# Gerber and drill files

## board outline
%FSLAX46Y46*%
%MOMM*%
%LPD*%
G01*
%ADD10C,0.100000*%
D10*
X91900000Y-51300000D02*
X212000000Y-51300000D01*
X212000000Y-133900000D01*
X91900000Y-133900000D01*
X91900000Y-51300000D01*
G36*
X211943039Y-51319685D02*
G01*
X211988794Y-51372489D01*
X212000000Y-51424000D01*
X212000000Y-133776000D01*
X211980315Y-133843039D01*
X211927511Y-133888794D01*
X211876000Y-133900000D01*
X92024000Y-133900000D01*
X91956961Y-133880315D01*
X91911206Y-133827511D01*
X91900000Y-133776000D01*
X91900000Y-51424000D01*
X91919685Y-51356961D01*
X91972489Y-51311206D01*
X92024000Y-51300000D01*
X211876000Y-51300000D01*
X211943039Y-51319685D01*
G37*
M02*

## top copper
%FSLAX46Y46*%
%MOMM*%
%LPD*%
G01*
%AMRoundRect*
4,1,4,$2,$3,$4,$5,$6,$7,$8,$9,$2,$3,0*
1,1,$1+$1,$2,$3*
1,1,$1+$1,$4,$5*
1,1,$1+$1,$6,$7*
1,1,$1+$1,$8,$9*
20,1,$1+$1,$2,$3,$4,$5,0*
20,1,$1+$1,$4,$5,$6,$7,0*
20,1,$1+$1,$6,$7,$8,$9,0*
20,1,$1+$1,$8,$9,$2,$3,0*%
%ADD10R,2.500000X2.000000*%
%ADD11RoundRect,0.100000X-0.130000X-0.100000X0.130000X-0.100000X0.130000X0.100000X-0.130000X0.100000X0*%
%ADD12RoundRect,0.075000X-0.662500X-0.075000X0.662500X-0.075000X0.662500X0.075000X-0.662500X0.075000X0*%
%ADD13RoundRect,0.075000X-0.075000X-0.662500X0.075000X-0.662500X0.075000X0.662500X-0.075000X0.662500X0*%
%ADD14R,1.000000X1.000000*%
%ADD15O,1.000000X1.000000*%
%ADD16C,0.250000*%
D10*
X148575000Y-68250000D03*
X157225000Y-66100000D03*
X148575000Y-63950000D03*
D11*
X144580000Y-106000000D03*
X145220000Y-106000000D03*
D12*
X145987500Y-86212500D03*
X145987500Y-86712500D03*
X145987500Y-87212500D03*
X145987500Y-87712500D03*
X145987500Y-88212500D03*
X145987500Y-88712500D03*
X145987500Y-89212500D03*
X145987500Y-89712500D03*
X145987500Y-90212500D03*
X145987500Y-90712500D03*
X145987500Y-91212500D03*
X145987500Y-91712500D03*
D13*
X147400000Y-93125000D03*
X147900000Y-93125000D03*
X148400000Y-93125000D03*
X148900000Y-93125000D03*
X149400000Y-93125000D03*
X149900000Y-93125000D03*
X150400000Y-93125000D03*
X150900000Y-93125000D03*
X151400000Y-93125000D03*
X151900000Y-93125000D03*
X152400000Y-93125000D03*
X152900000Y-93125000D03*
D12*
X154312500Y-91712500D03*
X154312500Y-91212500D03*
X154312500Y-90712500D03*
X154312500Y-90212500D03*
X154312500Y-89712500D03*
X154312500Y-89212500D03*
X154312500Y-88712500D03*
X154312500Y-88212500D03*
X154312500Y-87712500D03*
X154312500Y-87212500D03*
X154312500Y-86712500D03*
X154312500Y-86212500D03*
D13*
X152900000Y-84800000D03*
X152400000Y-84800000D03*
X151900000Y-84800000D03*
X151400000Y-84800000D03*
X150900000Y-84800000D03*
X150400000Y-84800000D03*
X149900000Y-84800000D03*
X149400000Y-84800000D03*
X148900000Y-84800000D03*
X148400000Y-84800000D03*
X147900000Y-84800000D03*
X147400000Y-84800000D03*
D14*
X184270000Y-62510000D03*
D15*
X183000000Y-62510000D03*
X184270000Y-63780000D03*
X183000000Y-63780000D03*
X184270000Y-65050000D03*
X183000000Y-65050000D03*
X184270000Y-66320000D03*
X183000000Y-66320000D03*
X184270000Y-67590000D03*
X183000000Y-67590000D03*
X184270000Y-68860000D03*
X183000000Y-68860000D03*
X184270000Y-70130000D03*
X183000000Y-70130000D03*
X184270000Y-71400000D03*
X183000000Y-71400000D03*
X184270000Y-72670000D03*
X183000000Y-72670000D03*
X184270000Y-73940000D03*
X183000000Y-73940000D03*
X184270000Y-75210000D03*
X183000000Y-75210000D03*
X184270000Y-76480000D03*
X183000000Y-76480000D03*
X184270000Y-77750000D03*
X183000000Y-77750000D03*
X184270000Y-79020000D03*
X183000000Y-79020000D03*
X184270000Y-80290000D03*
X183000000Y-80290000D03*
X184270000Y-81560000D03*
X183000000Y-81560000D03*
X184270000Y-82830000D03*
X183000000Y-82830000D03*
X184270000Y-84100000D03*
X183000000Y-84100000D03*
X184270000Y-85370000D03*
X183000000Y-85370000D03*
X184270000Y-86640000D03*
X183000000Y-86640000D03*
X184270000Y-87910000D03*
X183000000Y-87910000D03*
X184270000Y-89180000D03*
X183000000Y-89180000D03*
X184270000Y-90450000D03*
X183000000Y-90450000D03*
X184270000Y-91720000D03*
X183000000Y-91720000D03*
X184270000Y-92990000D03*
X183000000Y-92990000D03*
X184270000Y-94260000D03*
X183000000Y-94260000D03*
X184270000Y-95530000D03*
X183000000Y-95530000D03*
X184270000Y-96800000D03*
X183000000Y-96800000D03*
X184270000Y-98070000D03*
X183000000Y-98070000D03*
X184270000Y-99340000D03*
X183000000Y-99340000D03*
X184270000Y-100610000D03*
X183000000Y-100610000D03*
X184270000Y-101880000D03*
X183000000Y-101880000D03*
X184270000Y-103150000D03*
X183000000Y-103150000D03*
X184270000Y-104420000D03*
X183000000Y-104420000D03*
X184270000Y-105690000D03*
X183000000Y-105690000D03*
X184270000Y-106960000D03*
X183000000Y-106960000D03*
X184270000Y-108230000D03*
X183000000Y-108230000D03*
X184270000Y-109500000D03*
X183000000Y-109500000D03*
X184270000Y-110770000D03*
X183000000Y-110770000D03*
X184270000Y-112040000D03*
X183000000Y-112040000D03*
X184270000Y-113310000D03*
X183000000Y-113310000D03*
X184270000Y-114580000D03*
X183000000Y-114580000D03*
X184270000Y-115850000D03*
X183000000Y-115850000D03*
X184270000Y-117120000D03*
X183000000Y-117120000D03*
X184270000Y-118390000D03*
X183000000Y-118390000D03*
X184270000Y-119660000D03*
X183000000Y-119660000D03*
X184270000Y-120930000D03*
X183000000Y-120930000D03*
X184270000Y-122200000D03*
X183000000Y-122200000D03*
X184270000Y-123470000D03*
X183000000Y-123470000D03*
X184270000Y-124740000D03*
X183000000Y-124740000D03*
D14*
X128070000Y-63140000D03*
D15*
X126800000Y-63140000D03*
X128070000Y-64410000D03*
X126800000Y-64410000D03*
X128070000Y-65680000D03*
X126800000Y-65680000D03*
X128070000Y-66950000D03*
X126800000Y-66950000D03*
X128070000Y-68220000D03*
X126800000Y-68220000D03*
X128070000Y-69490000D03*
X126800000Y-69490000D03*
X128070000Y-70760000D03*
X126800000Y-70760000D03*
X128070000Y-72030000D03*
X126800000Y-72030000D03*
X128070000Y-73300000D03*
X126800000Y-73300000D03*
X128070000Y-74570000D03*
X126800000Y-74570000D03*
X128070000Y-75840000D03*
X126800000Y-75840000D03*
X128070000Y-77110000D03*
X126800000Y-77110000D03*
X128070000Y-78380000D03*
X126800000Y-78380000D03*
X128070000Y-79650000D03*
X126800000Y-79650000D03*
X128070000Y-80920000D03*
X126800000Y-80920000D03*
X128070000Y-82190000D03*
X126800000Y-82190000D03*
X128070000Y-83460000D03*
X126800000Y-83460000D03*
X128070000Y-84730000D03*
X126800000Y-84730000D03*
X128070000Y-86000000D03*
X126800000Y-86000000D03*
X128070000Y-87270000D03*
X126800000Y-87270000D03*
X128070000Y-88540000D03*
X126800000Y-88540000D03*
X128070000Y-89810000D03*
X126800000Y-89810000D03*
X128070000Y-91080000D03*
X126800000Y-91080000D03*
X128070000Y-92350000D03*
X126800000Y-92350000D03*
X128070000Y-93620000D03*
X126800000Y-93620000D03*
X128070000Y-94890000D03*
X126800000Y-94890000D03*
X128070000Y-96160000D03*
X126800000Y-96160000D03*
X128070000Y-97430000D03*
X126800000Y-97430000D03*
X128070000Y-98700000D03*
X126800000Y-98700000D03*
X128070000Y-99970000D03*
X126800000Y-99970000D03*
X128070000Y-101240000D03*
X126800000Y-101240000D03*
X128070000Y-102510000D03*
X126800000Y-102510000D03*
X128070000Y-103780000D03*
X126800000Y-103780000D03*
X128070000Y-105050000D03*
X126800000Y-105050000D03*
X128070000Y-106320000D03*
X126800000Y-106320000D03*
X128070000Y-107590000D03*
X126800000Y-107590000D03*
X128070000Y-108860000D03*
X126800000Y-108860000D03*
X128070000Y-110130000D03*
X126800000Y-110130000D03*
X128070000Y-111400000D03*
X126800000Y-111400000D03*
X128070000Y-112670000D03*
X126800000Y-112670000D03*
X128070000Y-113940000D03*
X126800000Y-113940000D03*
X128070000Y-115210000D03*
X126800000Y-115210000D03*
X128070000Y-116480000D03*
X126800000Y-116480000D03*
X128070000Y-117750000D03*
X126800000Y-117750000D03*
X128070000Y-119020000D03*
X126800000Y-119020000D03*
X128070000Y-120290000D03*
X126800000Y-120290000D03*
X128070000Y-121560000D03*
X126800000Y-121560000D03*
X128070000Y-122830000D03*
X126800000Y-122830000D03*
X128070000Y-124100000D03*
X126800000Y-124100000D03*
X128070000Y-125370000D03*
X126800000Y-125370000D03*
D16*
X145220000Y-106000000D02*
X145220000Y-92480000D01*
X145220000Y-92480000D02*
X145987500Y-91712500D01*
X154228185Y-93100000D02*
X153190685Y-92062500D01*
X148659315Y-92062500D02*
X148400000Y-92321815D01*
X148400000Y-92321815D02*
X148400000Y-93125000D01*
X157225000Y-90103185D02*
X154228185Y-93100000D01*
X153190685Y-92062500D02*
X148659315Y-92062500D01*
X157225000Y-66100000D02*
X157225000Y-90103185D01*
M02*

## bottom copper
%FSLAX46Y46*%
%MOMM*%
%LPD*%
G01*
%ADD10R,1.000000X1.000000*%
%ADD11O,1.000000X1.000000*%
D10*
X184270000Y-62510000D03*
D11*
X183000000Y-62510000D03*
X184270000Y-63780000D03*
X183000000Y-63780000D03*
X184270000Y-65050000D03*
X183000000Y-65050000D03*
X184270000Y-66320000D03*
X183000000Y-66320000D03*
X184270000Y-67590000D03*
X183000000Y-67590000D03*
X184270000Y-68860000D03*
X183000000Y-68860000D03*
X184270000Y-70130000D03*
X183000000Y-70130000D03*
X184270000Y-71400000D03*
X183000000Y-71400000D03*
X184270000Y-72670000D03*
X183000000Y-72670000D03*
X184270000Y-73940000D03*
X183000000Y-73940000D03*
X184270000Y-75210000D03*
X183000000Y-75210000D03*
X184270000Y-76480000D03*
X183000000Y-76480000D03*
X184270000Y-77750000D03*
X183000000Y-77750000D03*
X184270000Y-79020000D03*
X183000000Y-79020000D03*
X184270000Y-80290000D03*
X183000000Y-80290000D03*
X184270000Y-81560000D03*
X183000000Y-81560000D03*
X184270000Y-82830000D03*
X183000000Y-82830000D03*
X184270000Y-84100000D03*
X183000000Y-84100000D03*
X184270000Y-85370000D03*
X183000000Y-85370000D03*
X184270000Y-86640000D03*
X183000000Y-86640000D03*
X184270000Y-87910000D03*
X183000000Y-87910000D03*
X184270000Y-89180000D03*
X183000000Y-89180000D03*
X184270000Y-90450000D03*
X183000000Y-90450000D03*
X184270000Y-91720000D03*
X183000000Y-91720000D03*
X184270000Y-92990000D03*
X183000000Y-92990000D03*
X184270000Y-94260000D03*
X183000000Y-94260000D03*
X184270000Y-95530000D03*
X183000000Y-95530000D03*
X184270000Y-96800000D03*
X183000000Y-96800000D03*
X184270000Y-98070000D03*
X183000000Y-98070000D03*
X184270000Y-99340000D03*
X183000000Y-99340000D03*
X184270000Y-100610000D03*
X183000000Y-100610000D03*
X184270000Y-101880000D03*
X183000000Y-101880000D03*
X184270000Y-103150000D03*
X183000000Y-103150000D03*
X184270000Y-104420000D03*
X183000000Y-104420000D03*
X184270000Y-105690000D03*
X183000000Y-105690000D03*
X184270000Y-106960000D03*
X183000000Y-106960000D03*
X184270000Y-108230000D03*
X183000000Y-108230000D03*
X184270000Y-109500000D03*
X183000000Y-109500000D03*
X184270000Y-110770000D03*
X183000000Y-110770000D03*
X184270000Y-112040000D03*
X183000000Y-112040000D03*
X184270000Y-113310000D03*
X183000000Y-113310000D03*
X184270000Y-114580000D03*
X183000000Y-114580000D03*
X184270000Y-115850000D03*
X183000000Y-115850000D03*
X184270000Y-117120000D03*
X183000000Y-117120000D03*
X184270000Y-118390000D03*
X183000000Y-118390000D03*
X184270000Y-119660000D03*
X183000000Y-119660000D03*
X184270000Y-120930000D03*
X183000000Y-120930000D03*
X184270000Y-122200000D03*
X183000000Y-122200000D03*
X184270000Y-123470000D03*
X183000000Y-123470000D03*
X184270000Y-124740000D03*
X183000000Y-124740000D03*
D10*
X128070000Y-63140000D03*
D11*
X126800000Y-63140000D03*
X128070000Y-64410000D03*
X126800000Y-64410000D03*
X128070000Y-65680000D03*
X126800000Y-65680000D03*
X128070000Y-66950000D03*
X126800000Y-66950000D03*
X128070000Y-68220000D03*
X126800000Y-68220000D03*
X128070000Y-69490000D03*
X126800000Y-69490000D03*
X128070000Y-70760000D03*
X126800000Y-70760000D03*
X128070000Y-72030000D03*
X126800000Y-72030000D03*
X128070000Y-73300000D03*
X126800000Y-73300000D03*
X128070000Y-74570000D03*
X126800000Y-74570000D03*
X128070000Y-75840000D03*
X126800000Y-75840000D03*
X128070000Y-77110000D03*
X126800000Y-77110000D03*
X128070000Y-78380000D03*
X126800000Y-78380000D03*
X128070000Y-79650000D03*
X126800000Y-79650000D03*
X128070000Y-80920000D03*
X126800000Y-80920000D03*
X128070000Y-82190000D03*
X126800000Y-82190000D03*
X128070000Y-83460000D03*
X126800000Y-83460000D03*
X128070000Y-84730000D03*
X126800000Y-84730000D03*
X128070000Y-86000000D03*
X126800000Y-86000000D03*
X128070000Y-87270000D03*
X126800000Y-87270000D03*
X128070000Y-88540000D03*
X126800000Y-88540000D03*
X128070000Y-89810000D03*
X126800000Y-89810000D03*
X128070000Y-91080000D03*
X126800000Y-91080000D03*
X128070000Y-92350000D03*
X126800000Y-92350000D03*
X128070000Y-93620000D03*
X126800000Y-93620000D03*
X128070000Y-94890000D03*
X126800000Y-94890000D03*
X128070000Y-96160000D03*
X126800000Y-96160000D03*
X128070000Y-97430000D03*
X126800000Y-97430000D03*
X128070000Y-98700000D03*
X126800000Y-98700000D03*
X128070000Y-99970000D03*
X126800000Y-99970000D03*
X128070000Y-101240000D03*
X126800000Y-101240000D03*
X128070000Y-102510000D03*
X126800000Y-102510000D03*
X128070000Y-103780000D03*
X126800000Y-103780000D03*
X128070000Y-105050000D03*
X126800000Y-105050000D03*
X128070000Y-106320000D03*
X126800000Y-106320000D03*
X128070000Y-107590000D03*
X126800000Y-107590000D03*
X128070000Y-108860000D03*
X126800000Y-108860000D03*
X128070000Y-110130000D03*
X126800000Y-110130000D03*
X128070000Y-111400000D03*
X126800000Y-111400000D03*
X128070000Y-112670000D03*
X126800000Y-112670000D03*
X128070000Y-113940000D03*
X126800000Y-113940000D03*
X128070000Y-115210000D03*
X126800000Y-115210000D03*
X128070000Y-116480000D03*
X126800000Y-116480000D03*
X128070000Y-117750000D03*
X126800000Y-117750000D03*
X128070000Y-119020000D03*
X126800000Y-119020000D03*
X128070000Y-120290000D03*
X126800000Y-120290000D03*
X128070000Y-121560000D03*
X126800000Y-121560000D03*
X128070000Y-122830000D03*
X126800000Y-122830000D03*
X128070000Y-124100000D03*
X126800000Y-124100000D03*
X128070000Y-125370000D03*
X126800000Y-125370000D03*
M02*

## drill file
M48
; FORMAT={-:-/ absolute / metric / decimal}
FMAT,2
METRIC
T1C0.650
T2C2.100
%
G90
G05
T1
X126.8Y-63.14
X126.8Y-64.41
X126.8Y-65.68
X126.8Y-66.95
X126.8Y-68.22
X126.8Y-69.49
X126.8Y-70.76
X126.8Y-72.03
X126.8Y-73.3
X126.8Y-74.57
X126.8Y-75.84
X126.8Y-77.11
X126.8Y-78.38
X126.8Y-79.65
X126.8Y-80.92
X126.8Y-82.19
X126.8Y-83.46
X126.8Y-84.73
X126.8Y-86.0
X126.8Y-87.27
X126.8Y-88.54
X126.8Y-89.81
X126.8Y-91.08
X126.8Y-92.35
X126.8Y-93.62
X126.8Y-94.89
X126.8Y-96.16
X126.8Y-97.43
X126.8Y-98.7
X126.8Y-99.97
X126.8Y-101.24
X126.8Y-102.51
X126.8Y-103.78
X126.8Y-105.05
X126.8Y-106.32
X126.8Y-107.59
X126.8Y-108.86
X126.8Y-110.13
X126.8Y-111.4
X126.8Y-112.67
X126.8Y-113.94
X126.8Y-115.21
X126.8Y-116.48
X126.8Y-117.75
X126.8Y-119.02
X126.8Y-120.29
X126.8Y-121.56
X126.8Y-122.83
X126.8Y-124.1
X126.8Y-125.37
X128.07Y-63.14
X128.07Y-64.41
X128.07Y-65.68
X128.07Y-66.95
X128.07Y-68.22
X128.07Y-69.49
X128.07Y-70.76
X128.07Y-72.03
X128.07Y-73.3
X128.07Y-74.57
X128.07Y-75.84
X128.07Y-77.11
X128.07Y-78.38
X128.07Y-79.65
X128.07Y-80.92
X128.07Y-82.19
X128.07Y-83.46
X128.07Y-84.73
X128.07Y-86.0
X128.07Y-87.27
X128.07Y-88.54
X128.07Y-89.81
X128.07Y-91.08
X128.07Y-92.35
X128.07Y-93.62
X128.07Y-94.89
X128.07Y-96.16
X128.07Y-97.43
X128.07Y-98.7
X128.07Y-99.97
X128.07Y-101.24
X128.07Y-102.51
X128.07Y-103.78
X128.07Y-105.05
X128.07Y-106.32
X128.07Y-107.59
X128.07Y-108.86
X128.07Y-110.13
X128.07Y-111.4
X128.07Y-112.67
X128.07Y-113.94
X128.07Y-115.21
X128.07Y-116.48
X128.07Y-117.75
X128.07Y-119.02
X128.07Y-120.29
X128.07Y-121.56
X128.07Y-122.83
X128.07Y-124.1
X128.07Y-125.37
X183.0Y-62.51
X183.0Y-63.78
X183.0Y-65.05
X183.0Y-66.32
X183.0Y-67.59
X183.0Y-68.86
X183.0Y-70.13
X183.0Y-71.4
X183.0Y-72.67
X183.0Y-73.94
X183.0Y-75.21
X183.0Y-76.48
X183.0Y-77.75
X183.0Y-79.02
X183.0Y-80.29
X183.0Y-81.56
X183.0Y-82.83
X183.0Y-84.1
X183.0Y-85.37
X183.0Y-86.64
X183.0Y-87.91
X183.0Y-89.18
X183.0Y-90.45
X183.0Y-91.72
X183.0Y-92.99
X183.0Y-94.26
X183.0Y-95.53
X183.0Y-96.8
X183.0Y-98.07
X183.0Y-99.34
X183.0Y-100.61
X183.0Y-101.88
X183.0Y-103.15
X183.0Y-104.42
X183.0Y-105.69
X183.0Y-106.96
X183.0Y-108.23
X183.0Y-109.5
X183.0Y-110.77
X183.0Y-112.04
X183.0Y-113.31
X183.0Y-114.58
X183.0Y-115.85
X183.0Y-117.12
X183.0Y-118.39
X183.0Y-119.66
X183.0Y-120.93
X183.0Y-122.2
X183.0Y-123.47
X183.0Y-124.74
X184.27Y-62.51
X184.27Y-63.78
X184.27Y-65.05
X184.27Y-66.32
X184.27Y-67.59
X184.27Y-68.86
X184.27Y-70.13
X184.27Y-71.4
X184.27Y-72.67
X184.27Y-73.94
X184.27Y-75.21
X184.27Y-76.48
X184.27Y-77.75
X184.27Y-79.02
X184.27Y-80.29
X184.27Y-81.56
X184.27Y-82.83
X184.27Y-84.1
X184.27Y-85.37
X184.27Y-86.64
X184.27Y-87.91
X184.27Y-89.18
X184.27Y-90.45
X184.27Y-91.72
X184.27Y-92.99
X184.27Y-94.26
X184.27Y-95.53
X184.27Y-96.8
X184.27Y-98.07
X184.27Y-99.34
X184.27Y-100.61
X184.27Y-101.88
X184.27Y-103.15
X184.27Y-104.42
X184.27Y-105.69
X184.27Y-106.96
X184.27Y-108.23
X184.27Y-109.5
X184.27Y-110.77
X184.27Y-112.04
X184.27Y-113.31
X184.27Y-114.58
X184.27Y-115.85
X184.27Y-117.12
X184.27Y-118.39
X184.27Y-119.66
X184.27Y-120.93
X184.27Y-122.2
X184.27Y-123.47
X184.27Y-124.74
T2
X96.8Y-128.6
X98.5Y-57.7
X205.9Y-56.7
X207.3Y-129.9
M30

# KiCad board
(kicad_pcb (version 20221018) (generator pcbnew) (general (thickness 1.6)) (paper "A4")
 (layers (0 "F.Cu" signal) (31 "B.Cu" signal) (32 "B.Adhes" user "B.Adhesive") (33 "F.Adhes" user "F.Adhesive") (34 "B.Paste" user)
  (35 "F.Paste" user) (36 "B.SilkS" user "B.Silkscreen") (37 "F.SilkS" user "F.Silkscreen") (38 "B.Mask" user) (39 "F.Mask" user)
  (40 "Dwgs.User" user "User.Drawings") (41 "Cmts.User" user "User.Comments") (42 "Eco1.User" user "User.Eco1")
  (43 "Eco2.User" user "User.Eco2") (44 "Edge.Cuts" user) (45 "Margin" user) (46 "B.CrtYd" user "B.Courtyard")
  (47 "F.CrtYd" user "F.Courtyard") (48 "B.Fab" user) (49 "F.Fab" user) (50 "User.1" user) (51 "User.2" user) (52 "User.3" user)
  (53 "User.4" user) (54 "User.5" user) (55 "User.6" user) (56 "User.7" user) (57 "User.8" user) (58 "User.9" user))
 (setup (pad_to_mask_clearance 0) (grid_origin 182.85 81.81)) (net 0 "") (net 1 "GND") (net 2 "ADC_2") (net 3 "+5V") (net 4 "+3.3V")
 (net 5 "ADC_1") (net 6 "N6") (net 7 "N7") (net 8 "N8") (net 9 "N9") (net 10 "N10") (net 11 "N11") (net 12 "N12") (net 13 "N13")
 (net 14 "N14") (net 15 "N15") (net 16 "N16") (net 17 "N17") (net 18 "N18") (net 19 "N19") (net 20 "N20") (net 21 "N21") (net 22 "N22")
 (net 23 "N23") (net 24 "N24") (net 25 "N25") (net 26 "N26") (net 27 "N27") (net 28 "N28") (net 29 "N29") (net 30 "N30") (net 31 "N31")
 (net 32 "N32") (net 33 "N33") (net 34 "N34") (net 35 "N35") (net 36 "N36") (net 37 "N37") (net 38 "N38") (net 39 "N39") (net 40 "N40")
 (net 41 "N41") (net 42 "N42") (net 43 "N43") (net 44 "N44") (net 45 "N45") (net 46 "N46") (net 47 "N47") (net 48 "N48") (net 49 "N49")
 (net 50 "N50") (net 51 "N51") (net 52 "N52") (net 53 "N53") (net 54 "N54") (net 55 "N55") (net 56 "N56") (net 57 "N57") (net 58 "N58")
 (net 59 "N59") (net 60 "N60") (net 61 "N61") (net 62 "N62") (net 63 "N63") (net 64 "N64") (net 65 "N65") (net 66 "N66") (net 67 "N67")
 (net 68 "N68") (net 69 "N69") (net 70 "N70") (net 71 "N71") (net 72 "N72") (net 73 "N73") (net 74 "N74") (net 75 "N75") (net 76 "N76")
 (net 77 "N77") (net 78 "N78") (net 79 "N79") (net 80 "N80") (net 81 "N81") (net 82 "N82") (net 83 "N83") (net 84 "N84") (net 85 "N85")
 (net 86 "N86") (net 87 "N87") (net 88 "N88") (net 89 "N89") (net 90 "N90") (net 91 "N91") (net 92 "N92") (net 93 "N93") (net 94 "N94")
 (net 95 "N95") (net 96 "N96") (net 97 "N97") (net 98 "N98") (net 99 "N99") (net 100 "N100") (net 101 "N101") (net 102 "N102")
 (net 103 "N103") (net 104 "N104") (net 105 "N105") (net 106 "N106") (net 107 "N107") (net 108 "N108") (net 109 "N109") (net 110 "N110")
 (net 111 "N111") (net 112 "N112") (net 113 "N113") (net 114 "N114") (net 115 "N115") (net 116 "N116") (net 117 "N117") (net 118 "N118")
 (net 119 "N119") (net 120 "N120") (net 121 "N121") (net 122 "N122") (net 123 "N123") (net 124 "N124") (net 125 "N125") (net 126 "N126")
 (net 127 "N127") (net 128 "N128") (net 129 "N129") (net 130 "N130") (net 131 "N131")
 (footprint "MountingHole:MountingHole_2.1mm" (layer "F.Cu") (at 96.8 128.6)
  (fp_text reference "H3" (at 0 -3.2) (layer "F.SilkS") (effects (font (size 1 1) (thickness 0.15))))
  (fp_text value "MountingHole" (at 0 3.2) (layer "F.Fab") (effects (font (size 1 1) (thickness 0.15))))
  (pad "" np_thru_hole circle (at 0 0) (size 2.1 2.1) (drill 2.1) (layers "*.Cu" "*.Mask")))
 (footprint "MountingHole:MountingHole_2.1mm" (layer "F.Cu") (at 98.5 57.7)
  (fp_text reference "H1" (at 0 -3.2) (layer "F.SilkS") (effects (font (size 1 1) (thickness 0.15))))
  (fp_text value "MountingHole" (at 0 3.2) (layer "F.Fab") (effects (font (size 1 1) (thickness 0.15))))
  (pad "" np_thru_hole circle (at 0 0) (size 2.1 2.1) (drill 2.1) (layers "*.Cu" "*.Mask")))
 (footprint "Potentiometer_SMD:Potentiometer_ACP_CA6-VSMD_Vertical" (layer "F.Cu") (at 152.9 66.1)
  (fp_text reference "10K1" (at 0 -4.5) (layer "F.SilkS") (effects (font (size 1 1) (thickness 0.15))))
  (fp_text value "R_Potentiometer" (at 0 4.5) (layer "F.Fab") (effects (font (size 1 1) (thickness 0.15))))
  (pad "1" smd rect (at -4.325 2.15) (size 2.5 2) (layers "F.Cu" "F.Paste" "F.Mask") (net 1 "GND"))
  (pad "2" smd rect (at 4.325 0) (size 2.5 2) (layers "F.Cu" "F.Paste" "F.Mask") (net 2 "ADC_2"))
  (pad "3" smd rect (at -4.325 -2.15) (size 2.5 2) (layers "F.Cu" "F.Paste" "F.Mask") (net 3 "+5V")))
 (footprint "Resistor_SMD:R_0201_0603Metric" (layer "F.Cu") (at 144.9 106)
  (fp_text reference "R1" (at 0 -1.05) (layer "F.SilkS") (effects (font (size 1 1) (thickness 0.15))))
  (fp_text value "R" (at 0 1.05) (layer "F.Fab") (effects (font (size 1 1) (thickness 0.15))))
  (pad "" smd roundrect (at -0.345 0) (size 0.318 0.36) (layers "F.Paste") (roundrect_rratio 0.25))
  (pad "" smd roundrect (at 0.345 0) (size 0.318 0.36) (layers "F.Paste") (roundrect_rratio 0.25))
  (pad "1" smd roundrect (at -0.32 0) (size 0.46 0.4) (layers "F.Cu" "F.Mask") (roundrect_rratio 0.25) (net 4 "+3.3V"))
  (pad "2" smd roundrect (at 0.32 0) (size 0.46 0.4) (layers "F.Cu" "F.Mask") (roundrect_rratio 0.25) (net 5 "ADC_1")))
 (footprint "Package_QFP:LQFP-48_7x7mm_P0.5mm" (layer "F.Cu") (at 150.15 88.9625)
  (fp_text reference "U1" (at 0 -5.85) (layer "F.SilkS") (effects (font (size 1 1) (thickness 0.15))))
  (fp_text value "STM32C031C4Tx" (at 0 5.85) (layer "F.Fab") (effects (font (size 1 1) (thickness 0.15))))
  (pad "1" smd roundrect (at -4.1625 -2.75) (size 1.475 0.3) (layers "F.Cu" "F.Paste" "F.Mask") (roundrect_rratio 0.25) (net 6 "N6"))
  (pad "2" smd roundrect (at -4.1625 -2.25) (size 1.475 0.3) (layers "F.Cu" "F.Paste" "F.Mask") (roundrect_rratio 0.25) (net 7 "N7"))
  (pad "3" smd roundrect (at -4.1625 -1.75) (size 1.475 0.3) (layers "F.Cu" "F.Paste" "F.Mask") (roundrect_rratio 0.25) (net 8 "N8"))
  (pad "4" smd roundrect (at -4.1625 -1.25) (size 1.475 0.3) (layers "F.Cu" "F.Paste" "F.Mask") (roundrect_rratio 0.25) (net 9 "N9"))
  (pad "5" smd roundrect (at -4.1625 -0.75) (size 1.475 0.3) (layers "F.Cu" "F.Paste" "F.Mask") (roundrect_rratio 0.25) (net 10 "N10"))
  (pad "6" smd roundrect (at -4.1625 -0.25) (size 1.475 0.3) (layers "F.Cu" "F.Paste" "F.Mask") (roundrect_rratio 0.25) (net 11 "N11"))
  (pad "7" smd roundrect (at -4.1625 0.25) (size 1.475 0.3) (layers "F.Cu" "F.Paste" "F.Mask") (roundrect_rratio 0.25) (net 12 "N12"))
  (pad "8" smd roundrect (at -4.1625 0.75) (size 1.475 0.3) (layers "F.Cu" "F.Paste" "F.Mask") (roundrect_rratio 0.25) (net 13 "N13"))
  (pad "9" smd roundrect (at -4.1625 1.25) (size 1.475 0.3) (layers "F.Cu" "F.Paste" "F.Mask") (roundrect_rratio 0.25) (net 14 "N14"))
  (pad "10" smd roundrect (at -4.1625 1.75) (size 1.475 0.3) (layers "F.Cu" "F.Paste" "F.Mask") (roundrect_rratio 0.25) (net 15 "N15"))
  (pad "11" smd roundrect (at -4.1625 2.25) (size 1.475 0.3) (layers "F.Cu" "F.Paste" "F.Mask") (roundrect_rratio 0.25) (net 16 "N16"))
  (pad "12" smd roundrect (at -4.1625 2.75) (size 1.475 0.3) (layers "F.Cu" "F.Paste" "F.Mask") (roundrect_rratio 0.25) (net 5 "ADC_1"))
  (pad "13" smd roundrect (at -2.75 4.1625) (size 0.3 1.475) (layers "F.Cu" "F.Paste" "F.Mask") (roundrect_rratio 0.25) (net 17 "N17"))
  (pad "14" smd roundrect (at -2.25 4.1625) (size 0.3 1.475) (layers "F.Cu" "F.Paste" "F.Mask") (roundrect_rratio 0.25) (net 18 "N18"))
  (pad "15" smd roundrect (at -1.75 4.1625) (size 0.3 1.475) (layers "F.Cu" "F.Paste" "F.Mask") (roundrect_rratio 0.25) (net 2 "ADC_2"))
  (pad "16" smd roundrect (at -1.25 4.1625) (size 0.3 1.475) (layers "F.Cu" "F.Paste" "F.Mask") (roundrect_rratio 0.25) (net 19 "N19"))
  (pad "17" smd roundrect (at -0.75 4.1625) (size 0.3 1.475) (layers "F.Cu" "F.Paste" "F.Mask") (roundrect_rratio 0.25) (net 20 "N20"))
  (pad "18" smd roundrect (at -0.25 4.1625) (size 0.3 1.475) (layers "F.Cu" "F.Paste" "F.Mask") (roundrect_rratio 0.25) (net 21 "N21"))
  (pad "19" smd roundrect (at 0.25 4.1625) (size 0.3 1.475) (layers "F.Cu" "F.Paste" "F.Mask") (roundrect_rratio 0.25) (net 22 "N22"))
  (pad "20" smd roundrect (at 0.75 4.1625) (size 0.3 1.475) (layers "F.Cu" "F.Paste" "F.Mask") (roundrect_rratio 0.25) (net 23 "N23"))
  (pad "21" smd roundrect (at 1.25 4.1625) (size 0.3 1.475) (layers "F.Cu" "F.Paste" "F.Mask") (roundrect_rratio 0.25) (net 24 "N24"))
  (pad "22" smd roundrect (at 1.75 4.1625) (size 0.3 1.475) (layers "F.Cu" "F.Paste" "F.Mask") (roundrect_rratio 0.25) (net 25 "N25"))
  (pad "23" smd roundrect (at 2.25 4.1625) (size 0.3 1.475) (layers "F.Cu" "F.Paste" "F.Mask") (roundrect_rratio 0.25) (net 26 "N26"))
  (pad "24" smd roundrect (at 2.75 4.1625) (size 0.3 1.475) (layers "F.Cu" "F.Paste" "F.Mask") (roundrect_rratio 0.25) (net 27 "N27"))
  (pad "25" smd roundrect (at 4.1625 2.75) (size 1.475 0.3) (layers "F.Cu" "F.Paste" "F.Mask") (roundrect_rratio 0.25) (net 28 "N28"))
  (pad "26" smd roundrect (at 4.1625 2.25) (size 1.475 0.3) (layers "F.Cu" "F.Paste" "F.Mask") (roundrect_rratio 0.25) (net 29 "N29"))
  (pad "27" smd roundrect (at 4.1625 1.75) (size 1.475 0.3) (layers "F.Cu" "F.Paste" "F.Mask") (roundrect_rratio 0.25) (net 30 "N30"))
  (pad "28" smd roundrect (at 4.1625 1.25) (size 1.475 0.3) (layers "F.Cu" "F.Paste" "F.Mask") (roundrect_rratio 0.25) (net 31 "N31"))
  (pad "29" smd roundrect (at 4.1625 0.75) (size 1.475 0.3) (layers "F.Cu" "F.Paste" "F.Mask") (roundrect_rratio 0.25) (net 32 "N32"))
  (pad "30" smd roundrect (at 4.1625 0.25) (size 1.475 0.3) (layers "F.Cu" "F.Paste" "F.Mask") (roundrect_rratio 0.25) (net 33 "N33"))
  (pad "31" smd roundrect (at 4.1625 -0.25) (size 1.475 0.3) (layers "F.Cu" "F.Paste" "F.Mask") (roundrect_rratio 0.25) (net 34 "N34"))
  (pad "32" smd roundrect (at 4.1625 -0.75) (size 1.475 0.3) (layers "F.Cu" "F.Paste" "F.Mask") (roundrect_rratio 0.25) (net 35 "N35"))
  (pad "33" smd roundrect (at 4.1625 -1.25) (size 1.475 0.3) (layers "F.Cu" "F.Paste" "F.Mask") (roundrect_rratio 0.25) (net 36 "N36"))
  (pad "34" smd roundrect (at 4.1625 -1.75) (size 1.475 0.3) (layers "F.Cu" "F.Paste" "F.Mask") (roundrect_rratio 0.25) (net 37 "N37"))
  (pad "35" smd roundrect (at 4.1625 -2.25) (size 1.475 0.3) (layers "F.Cu" "F.Paste" "F.Mask") (roundrect_rratio 0.25) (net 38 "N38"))
  (pad "36" smd roundrect (at 4.1625 -2.75) (size 1.475 0.3) (layers "F.Cu" "F.Paste" "F.Mask") (roundrect_rratio 0.25) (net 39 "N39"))
  (pad "37" smd roundrect (at 2.75 -4.1625) (size 0.3 1.475) (layers "F.Cu" "F.Paste" "F.Mask") (roundrect_rratio 0.25) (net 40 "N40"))
  (pad "38" smd roundrect (at 2.25 -4.1625) (size 0.3 1.475) (layers "F.Cu" "F.Paste" "F.Mask") (roundrect_rratio 0.25) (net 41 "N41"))
  (pad "39" smd roundrect (at 1.75 -4.1625) (size 0.3 1.475) (layers "F.Cu" "F.Paste" "F.Mask") (roundrect_rratio 0.25) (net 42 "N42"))
  (pad "40" smd roundrect (at 1.25 -4.1625) (size 0.3 1.475) (layers "F.Cu" "F.Paste" "F.Mask") (roundrect_rratio 0.25) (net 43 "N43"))
  (pad "41" smd roundrect (at 0.75 -4.1625) (size 0.3 1.475) (layers "F.Cu" "F.Paste" "F.Mask") (roundrect_rratio 0.25) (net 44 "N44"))
  (pad "42" smd roundrect (at 0.25 -4.1625) (size 0.3 1.475) (layers "F.Cu" "F.Paste" "F.Mask") (roundrect_rratio 0.25) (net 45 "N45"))
  (pad "43" smd roundrect (at -0.25 -4.1625) (size 0.3 1.475) (layers "F.Cu" "F.Paste" "F.Mask") (roundrect_rratio 0.25) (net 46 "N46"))
  (pad "44" smd roundrect (at -0.75 -4.1625) (size 0.3 1.475) (layers "F.Cu" "F.Paste" "F.Mask") (roundrect_rratio 0.25) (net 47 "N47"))
  (pad "45" smd roundrect (at -1.25 -4.1625) (size 0.3 1.475) (layers "F.Cu" "F.Paste" "F.Mask") (roundrect_rratio 0.25) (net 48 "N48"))
  (pad "46" smd roundrect (at -1.75 -4.1625) (size 0.3 1.475) (layers "F.Cu" "F.Paste" "F.Mask") (roundrect_rratio 0.25) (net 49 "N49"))
  (pad "47" smd roundrect (at -2.25 -4.1625) (size 0.3 1.475) (layers "F.Cu" "F.Paste" "F.Mask") (roundrect_rratio 0.25) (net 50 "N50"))
  (pad "48" smd roundrect (at -2.75 -4.1625) (size 0.3 1.475) (layers "F.Cu" "F.Paste" "F.Mask") (roundrect_rratio 0.25) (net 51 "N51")))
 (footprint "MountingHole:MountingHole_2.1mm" (layer "F.Cu") (at 207.3 129.9)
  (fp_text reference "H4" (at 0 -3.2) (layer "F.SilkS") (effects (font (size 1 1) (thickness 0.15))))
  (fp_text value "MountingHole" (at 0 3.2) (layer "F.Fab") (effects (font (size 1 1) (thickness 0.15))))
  (pad "" np_thru_hole circle (at 0 0) (size 2.1 2.1) (drill 2.1) (layers "*.Cu" "*.Mask")))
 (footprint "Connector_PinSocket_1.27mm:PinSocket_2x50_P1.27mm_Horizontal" (layer "F.Cu") (at 184.27 62.51)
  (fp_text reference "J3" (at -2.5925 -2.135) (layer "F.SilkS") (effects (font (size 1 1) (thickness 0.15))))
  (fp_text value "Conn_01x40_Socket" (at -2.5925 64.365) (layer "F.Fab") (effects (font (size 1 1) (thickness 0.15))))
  (pad "1" thru_hole rect (at 0 0) (size 1 1) (drill 0.65) (layers "*.Cu" "*.Mask") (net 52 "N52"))
  (pad "2" thru_hole oval (at -1.27 0) (size 1 1) (drill 0.65) (layers "*.Cu" "*.Mask") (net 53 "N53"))
  (pad "3" thru_hole oval (at 0 1.27) (size 1 1) (drill 0.65) (layers "*.Cu" "*.Mask") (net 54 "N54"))
  (pad "4" thru_hole oval (at -1.27 1.27) (size 1 1) (drill 0.65) (layers "*.Cu" "*.Mask") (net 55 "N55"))
  (pad "5" thru_hole oval (at 0 2.54) (size 1 1) (drill 0.65) (layers "*.Cu" "*.Mask") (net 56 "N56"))
  (pad "6" thru_hole oval (at -1.27 2.54) (size 1 1) (drill 0.65) (layers "*.Cu" "*.Mask") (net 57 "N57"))
  (pad "7" thru_hole oval (at 0 3.81) (size 1 1) (drill 0.65) (layers "*.Cu" "*.Mask") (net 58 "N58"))
  (pad "8" thru_hole oval (at -1.27 3.81) (size 1 1) (drill 0.65) (layers "*.Cu" "*.Mask") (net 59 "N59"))
  (pad "9" thru_hole oval (at 0 5.08) (size 1 1) (drill 0.65) (layers "*.Cu" "*.Mask") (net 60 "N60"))
  (pad "10" thru_hole oval (at -1.27 5.08) (size 1 1) (drill 0.65) (layers "*.Cu" "*.Mask") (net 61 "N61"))
  (pad "11" thru_hole oval (at 0 6.35) (size 1 1) (drill 0.65) (layers "*.Cu" "*.Mask") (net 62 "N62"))
  (pad "12" thru_hole oval (at -1.27 6.35) (size 1 1) (drill 0.65) (layers "*.Cu" "*.Mask") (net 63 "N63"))
  (pad "13" thru_hole oval (at 0 7.62) (size 1 1) (drill 0.65) (layers "*.Cu" "*.Mask") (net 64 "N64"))
  (pad "14" thru_hole oval (at -1.27 7.62) (size 1 1) (drill 0.65) (layers "*.Cu" "*.Mask") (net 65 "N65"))
  (pad "15" thru_hole oval (at 0 8.89) (size 1 1) (drill 0.65) (layers "*.Cu" "*.Mask") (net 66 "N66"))
  (pad "16" thru_hole oval (at -1.27 8.89) (size 1 1) (drill 0.65) (layers "*.Cu" "*.Mask") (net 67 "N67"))
  (pad "17" thru_hole oval (at 0 10.16) (size 1 1) (drill 0.65) (layers "*.Cu" "*.Mask") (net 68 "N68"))
  (pad "18" thru_hole oval (at -1.27 10.16) (size 1 1) (drill 0.65) (layers "*.Cu" "*.Mask") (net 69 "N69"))
  (pad "19" thru_hole oval (at 0 11.43) (size 1 1) (drill 0.65) (layers "*.Cu" "*.Mask") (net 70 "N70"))
  (pad "20" thru_hole oval (at -1.27 11.43) (size 1 1) (drill 0.65) (layers "*.Cu" "*.Mask") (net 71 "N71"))
  (pad "21" thru_hole oval (at 0 12.7) (size 1 1) (drill 0.65) (layers "*.Cu" "*.Mask") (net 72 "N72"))
  (pad "22" thru_hole oval (at -1.27 12.7) (size 1 1) (drill 0.65) (layers "*.Cu" "*.Mask") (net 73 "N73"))
  (pad "23" thru_hole oval (at 0 13.97) (size 1 1) (drill 0.65) (layers "*.Cu" "*.Mask") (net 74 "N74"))
  (pad "24" thru_hole oval (at -1.27 13.97) (size 1 1) (drill 0.65) (layers "*.Cu" "*.Mask") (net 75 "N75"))
  (pad "25" thru_hole oval (at 0 15.24) (size 1 1) (drill 0.65) (layers "*.Cu" "*.Mask") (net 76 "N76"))
  (pad "26" thru_hole oval (at -1.27 15.24) (size 1 1) (drill 0.65) (layers "*.Cu" "*.Mask") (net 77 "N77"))
  (pad "27" thru_hole oval (at 0 16.51) (size 1 1) (drill 0.65) (layers "*.Cu" "*.Mask") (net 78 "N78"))
  (pad "28" thru_hole oval (at -1.27 16.51) (size 1 1) (drill 0.65) (layers "*.Cu" "*.Mask") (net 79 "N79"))
  (pad "29" thru_hole oval (at 0 17.78) (size 1 1) (drill 0.65) (layers "*.Cu" "*.Mask") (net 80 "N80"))
  (pad "30" thru_hole oval (at -1.27 17.78) (size 1 1) (drill 0.65) (layers "*.Cu" "*.Mask") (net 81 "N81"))
  (pad "31" thru_hole oval (at 0 19.05) (size 1 1) (drill 0.65) (layers "*.Cu" "*.Mask") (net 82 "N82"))
  (pad "32" thru_hole oval (at -1.27 19.05) (size 1 1) (drill 0.65) (layers "*.Cu" "*.Mask") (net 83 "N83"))
  (pad "33" thru_hole oval (at 0 20.32) (size 1 1) (drill 0.65) (layers "*.Cu" "*.Mask") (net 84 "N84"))
  (pad "34" thru_hole oval (at -1.27 20.32) (size 1 1) (drill 0.65) (layers "*.Cu" "*.Mask") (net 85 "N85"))
  (pad "35" thru_hole oval (at 0 21.59) (size 1 1) (drill 0.65) (layers "*.Cu" "*.Mask") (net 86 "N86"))
  (pad "36" thru_hole oval (at -1.27 21.59) (size 1 1) (drill 0.65) (layers "*.Cu" "*.Mask") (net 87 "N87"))
  (pad "37" thru_hole oval (at 0 22.86) (size 1 1) (drill 0.65) (layers "*.Cu" "*.Mask") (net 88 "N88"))
  (pad "38" thru_hole oval (at -1.27 22.86) (size 1 1) (drill 0.65) (layers "*.Cu" "*.Mask") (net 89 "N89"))
  (pad "39" thru_hole oval (at 0 24.13) (size 1 1) (drill 0.65) (layers "*.Cu" "*.Mask") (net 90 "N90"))
  (pad "40" thru_hole oval (at -1.27 24.13) (size 1 1) (drill 0.65) (layers "*.Cu" "*.Mask") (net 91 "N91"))
  (pad "41" thru_hole oval (at 0 25.4) (size 1 1) (drill 0.65) (layers "*.Cu" "*.Mask"))
  (pad "42" thru_hole oval (at -1.27 25.4) (size 1 1) (drill 0.65) (layers "*.Cu" "*.Mask"))
  (pad "43" thru_hole oval (at 0 26.67) (size 1 1) (drill 0.65) (layers "*.Cu" "*.Mask"))
  (pad "44" thru_hole oval (at -1.27 26.67) (size 1 1) (drill 0.65) (layers "*.Cu" "*.Mask"))
  (pad "45" thru_hole oval (at 0 27.94) (size 1 1) (drill 0.65) (layers "*.Cu" "*.Mask"))
  (pad "46" thru_hole oval (at -1.27 27.94) (size 1 1) (drill 0.65) (layers "*.Cu" "*.Mask"))
  (pad "47" thru_hole oval (at 0 29.21) (size 1 1) (drill 0.65) (layers "*.Cu" "*.Mask"))
  (pad "48" thru_hole oval (at -1.27 29.21) (size 1 1) (drill 0.65) (layers "*.Cu" "*.Mask"))
  (pad "49" thru_hole oval (at 0 30.48) (size 1 1) (drill 0.65) (layers "*.Cu" "*.Mask"))
  (pad "50" thru_hole oval (at -1.27 30.48) (size 1 1) (drill 0.65) (layers "*.Cu" "*.Mask"))
  (pad "51" thru_hole oval (at 0 31.75) (size 1 1) (drill 0.65) (layers "*.Cu" "*.Mask"))
  (pad "52" thru_hole oval (at -1.27 31.75) (size 1 1) (drill 0.65) (layers "*.Cu" "*.Mask"))
  (pad "53" thru_hole oval (at 0 33.02) (size 1 1) (drill 0.65) (layers "*.Cu" "*.Mask"))
  (pad "54" thru_hole oval (at -1.27 33.02) (size 1 1) (drill 0.65) (layers "*.Cu" "*.Mask"))
  (pad "55" thru_hole oval (at 0 34.29) (size 1 1) (drill 0.65) (layers "*.Cu" "*.Mask"))
  (pad "56" thru_hole oval (at -1.27 34.29) (size 1 1) (drill 0.65) (layers "*.Cu" "*.Mask"))
  (pad "57" thru_hole oval (at 0 35.56) (size 1 1) (drill 0.65) (layers "*.Cu" "*.Mask"))
  (pad "58" thru_hole oval (at -1.27 35.56) (size 1 1) (drill 0.65) (layers "*.Cu" "*.Mask"))
  (pad "59" thru_hole oval (at 0 36.83) (size 1 1) (drill 0.65) (layers "*.Cu" "*.Mask"))
  (pad "60" thru_hole oval (at -1.27 36.83) (size 1 1) (drill 0.65) (layers "*.Cu" "*.Mask"))
  (pad "61" thru_hole oval (at 0 38.1) (size 1 1) (drill 0.65) (layers "*.Cu" "*.Mask"))
  (pad "62" thru_hole oval (at -1.27 38.1) (size 1 1) (drill 0.65) (layers "*.Cu" "*.Mask"))
  (pad "63" thru_hole oval (at 0 39.37) (size 1 1) (drill 0.65) (layers "*.Cu" "*.Mask"))
  (pad "64" thru_hole oval (at -1.27 39.37) (size 1 1) (drill 0.65) (layers "*.Cu" "*.Mask"))
  (pad "65" thru_hole oval (at 0 40.64) (size 1 1) (drill 0.65) (layers "*.Cu" "*.Mask"))
  (pad "66" thru_hole oval (at -1.27 40.64) (size 1 1) (drill 0.65) (layers "*.Cu" "*.Mask"))
  (pad "67" thru_hole oval (at 0 41.91) (size 1 1) (drill 0.65) (layers "*.Cu" "*.Mask"))
  (pad "68" thru_hole oval (at -1.27 41.91) (size 1 1) (drill 0.65) (layers "*.Cu" "*.Mask"))
  (pad "69" thru_hole oval (at 0 43.18) (size 1 1) (drill 0.65) (layers "*.Cu" "*.Mask"))
  (pad "70" thru_hole oval (at -1.27 43.18) (size 1 1) (drill 0.65) (layers "*.Cu" "*.Mask"))
  (pad "71" thru_hole oval (at 0 44.45) (size 1 1) (drill 0.65) (layers "*.Cu" "*.Mask"))
  (pad "72" thru_hole oval (at -1.27 44.45) (size 1 1) (drill 0.65) (layers "*.Cu" "*.Mask"))
  (pad "73" thru_hole oval (at 0 45.72) (size 1 1) (drill 0.65) (layers "*.Cu" "*.Mask"))
  (pad "74" thru_hole oval (at -1.27 45.72) (size 1 1) (drill 0.65) (layers "*.Cu" "*.Mask"))
  (pad "75" thru_hole oval (at 0 46.99) (size 1 1) (drill 0.65) (layers "*.Cu" "*.Mask"))
  (pad "76" thru_hole oval (at -1.27 46.99) (size 1 1) (drill 0.65) (layers "*.Cu" "*.Mask"))
  (pad "77" thru_hole oval (at 0 48.26) (size 1 1) (drill 0.65) (layers "*.Cu" "*.Mask"))
  (pad "78" thru_hole oval (at -1.27 48.26) (size 1 1) (drill 0.65) (layers "*.Cu" "*.Mask"))
  (pad "79" thru_hole oval (at 0 49.53) (size 1 1) (drill 0.65) (layers "*.Cu" "*.Mask"))
  (pad "80" thru_hole oval (at -1.27 49.53) (size 1 1) (drill 0.65) (layers "*.Cu" "*.Mask"))
  (pad "81" thru_hole oval (at 0 50.8) (size 1 1) (drill 0.65) (layers "*.Cu" "*.Mask"))
  (pad "82" thru_hole oval (at -1.27 50.8) (size 1 1) (drill 0.65) (layers "*.Cu" "*.Mask"))
  (pad "83" thru_hole oval (at 0 52.07) (size 1 1) (drill 0.65) (layers "*.Cu" "*.Mask"))
  (pad "84" thru_hole oval (at -1.27 52.07) (size 1 1) (drill 0.65) (layers "*.Cu" "*.Mask"))
  (pad "85" thru_hole oval (at 0 53.34) (size 1 1) (drill 0.65) (layers "*.Cu" "*.Mask"))
  (pad "86" thru_hole oval (at -1.27 53.34) (size 1 1) (drill 0.65) (layers "*.Cu" "*.Mask"))
  (pad "87" thru_hole oval (at 0 54.61) (size 1 1) (drill 0.65) (layers "*.Cu" "*.Mask"))
  (pad "88" thru_hole oval (at -1.27 54.61) (size 1 1) (drill 0.65) (layers "*.Cu" "*.Mask"))
  (pad "89" thru_hole oval (at 0 55.88) (size 1 1) (drill 0.65) (layers "*.Cu" "*.Mask"))
  (pad "90" thru_hole oval (at -1.27 55.88) (size 1 1) (drill 0.65) (layers "*.Cu" "*.Mask"))
  (pad "91" thru_hole oval (at 0 57.15) (size 1 1) (drill 0.65) (layers "*.Cu" "*.Mask"))
  (pad "92" thru_hole oval (at -1.27 57.15) (size 1 1) (drill 0.65) (layers "*.Cu" "*.Mask"))
  (pad "93" thru_hole oval (at 0 58.42) (size 1 1) (drill 0.65) (layers "*.Cu" "*.Mask"))
  (pad "94" thru_hole oval (at -1.27 58.42) (size 1 1) (drill 0.65) (layers "*.Cu" "*.Mask"))
  (pad "95" thru_hole oval (at 0 59.69) (size 1 1) (drill 0.65) (layers "*.Cu" "*.Mask"))
  (pad "96" thru_hole oval (at -1.27 59.69) (size 1 1) (drill 0.65) (layers "*.Cu" "*.Mask"))
  (pad "97" thru_hole oval (at 0 60.96) (size 1 1) (drill 0.65) (layers "*.Cu" "*.Mask"))
  (pad "98" thru_hole oval (at -1.27 60.96) (size 1 1) (drill 0.65) (layers "*.Cu" "*.Mask"))
  (pad "99" thru_hole oval (at 0 62.23) (size 1 1) (drill 0.65) (layers "*.Cu" "*.Mask"))
  (pad "100" thru_hole oval (at -1.27 62.23) (size 1 1) (drill 0.65) (layers "*.Cu" "*.Mask")))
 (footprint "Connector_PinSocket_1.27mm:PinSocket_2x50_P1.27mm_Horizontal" (layer "F.Cu") (at 128.07 63.14)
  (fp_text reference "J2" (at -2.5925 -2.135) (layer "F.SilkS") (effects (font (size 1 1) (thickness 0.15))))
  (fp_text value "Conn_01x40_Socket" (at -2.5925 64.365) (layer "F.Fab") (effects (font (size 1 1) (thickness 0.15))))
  (pad "1" thru_hole rect (at 0 0) (size 1 1) (drill 0.65) (layers "*.Cu" "*.Mask") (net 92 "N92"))
  (pad "2" thru_hole oval (at -1.27 0) (size 1 1) (drill 0.65) (layers "*.Cu" "*.Mask") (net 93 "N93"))
  (pad "3" thru_hole oval (at 0 1.27) (size 1 1) (drill 0.65) (layers "*.Cu" "*.Mask") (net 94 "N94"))
  (pad "4" thru_hole oval (at -1.27 1.27) (size 1 1) (drill 0.65) (layers "*.Cu" "*.Mask") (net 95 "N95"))
  (pad "5" thru_hole oval (at 0 2.54) (size 1 1) (drill 0.65) (layers "*.Cu" "*.Mask") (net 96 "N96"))
  (pad "6" thru_hole oval (at -1.27 2.54) (size 1 1) (drill 0.65) (layers "*.Cu" "*.Mask") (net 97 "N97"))
  (pad "7" thru_hole oval (at 0 3.81) (size 1 1) (drill 0.65) (layers "*.Cu" "*.Mask") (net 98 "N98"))
  (pad "8" thru_hole oval (at -1.27 3.81) (size 1 1) (drill 0.65) (layers "*.Cu" "*.Mask") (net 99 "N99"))
  (pad "9" thru_hole oval (at 0 5.08) (size 1 1) (drill 0.65) (layers "*.Cu" "*.Mask") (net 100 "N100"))
  (pad "10" thru_hole oval (at -1.27 5.08) (size 1 1) (drill 0.65) (layers "*.Cu" "*.Mask") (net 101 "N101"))
  (pad "11" thru_hole oval (at 0 6.35) (size 1 1) (drill 0.65) (layers "*.Cu" "*.Mask") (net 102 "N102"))
  (pad "12" thru_hole oval (at -1.27 6.35) (size 1 1) (drill 0.65) (layers "*.Cu" "*.Mask") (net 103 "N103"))
  (pad "13" thru_hole oval (at 0 7.62) (size 1 1) (drill 0.65) (layers "*.Cu" "*.Mask") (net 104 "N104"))
  (pad "14" thru_hole oval (at -1.27 7.62) (size 1 1) (drill 0.65) (layers "*.Cu" "*.Mask") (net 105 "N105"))
  (pad "15" thru_hole oval (at 0 8.89) (size 1 1) (drill 0.65) (layers "*.Cu" "*.Mask") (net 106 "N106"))
  (pad "16" thru_hole oval (at -1.27 8.89) (size 1 1) (drill 0.65) (layers "*.Cu" "*.Mask") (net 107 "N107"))
  (pad "17" thru_hole oval (at 0 10.16) (size 1 1) (drill 0.65) (layers "*.Cu" "*.Mask") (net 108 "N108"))
  (pad "18" thru_hole oval (at -1.27 10.16) (size 1 1) (drill 0.65) (layers "*.Cu" "*.Mask") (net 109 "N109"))
  (pad "19" thru_hole oval (at 0 11.43) (size 1 1) (drill 0.65) (layers "*.Cu" "*.Mask") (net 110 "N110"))
  (pad "20" thru_hole oval (at -1.27 11.43) (size 1 1) (drill 0.65) (layers "*.Cu" "*.Mask") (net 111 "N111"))
  (pad "21" thru_hole oval (at 0 12.7) (size 1 1) (drill 0.65) (layers "*.Cu" "*.Mask") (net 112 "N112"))
  (pad "22" thru_hole oval (at -1.27 12.7) (size 1 1) (drill 0.65) (layers "*.Cu" "*.Mask") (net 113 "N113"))
  (pad "23" thru_hole oval (at 0 13.97) (size 1 1) (drill 0.65) (layers "*.Cu" "*.Mask") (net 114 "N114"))
  (pad "24" thru_hole oval (at -1.27 13.97) (size 1 1) (drill 0.65) (layers "*.Cu" "*.Mask") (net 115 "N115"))
  (pad "25" thru_hole oval (at 0 15.24) (size 1 1) (drill 0.65) (layers "*.Cu" "*.Mask") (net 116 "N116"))
  (pad "26" thru_hole oval (at -1.27 15.24) (size 1 1) (drill 0.65) (layers "*.Cu" "*.Mask") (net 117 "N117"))
  (pad "27" thru_hole oval (at 0 16.51) (size 1 1) (drill 0.65) (layers "*.Cu" "*.Mask") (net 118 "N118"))
  (pad "28" thru_hole oval (at -1.27 16.51) (size 1 1) (drill 0.65) (layers "*.Cu" "*.Mask") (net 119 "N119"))
  (pad "29" thru_hole oval (at 0 17.78) (size 1 1) (drill 0.65) (layers "*.Cu" "*.Mask") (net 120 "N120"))
  (pad "30" thru_hole oval (at -1.27 17.78) (size 1 1) (drill 0.65) (layers "*.Cu" "*.Mask") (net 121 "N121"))
  (pad "31" thru_hole oval (at 0 19.05) (size 1 1) (drill 0.65) (layers "*.Cu" "*.Mask") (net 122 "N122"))
  (pad "32" thru_hole oval (at -1.27 19.05) (size 1 1) (drill 0.65) (layers "*.Cu" "*.Mask") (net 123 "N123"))
  (pad "33" thru_hole oval (at 0 20.32) (size 1 1) (drill 0.65) (layers "*.Cu" "*.Mask") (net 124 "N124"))
  (pad "34" thru_hole oval (at -1.27 20.32) (size 1 1) (drill 0.65) (layers "*.Cu" "*.Mask") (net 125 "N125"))
  (pad "35" thru_hole oval (at 0 21.59) (size 1 1) (drill 0.65) (layers "*.Cu" "*.Mask") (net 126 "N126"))
  (pad "36" thru_hole oval (at -1.27 21.59) (size 1 1) (drill 0.65) (layers "*.Cu" "*.Mask") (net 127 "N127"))
  (pad "37" thru_hole oval (at 0 22.86) (size 1 1) (drill 0.65) (layers "*.Cu" "*.Mask") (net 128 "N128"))
  (pad "38" thru_hole oval (at -1.27 22.86) (size 1 1) (drill 0.65) (layers "*.Cu" "*.Mask") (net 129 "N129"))
  (pad "39" thru_hole oval (at 0 24.13) (size 1 1) (drill 0.65) (layers "*.Cu" "*.Mask") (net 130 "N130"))
  (pad "40" thru_hole oval (at -1.27 24.13) (size 1 1) (drill 0.65) (layers "*.Cu" "*.Mask") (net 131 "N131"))
  (pad "41" thru_hole oval (at 0 25.4) (size 1 1) (drill 0.65) (layers "*.Cu" "*.Mask"))
  (pad "42" thru_hole oval (at -1.27 25.4) (size 1 1) (drill 0.65) (layers "*.Cu" "*.Mask"))
  (pad "43" thru_hole oval (at 0 26.67) (size 1 1) (drill 0.65) (layers "*.Cu" "*.Mask"))
  (pad "44" thru_hole oval (at -1.27 26.67) (size 1 1) (drill 0.65) (layers "*.Cu" "*.Mask"))
  (pad "45" thru_hole oval (at 0 27.94) (size 1 1) (drill 0.65) (layers "*.Cu" "*.Mask"))
  (pad "46" thru_hole oval (at -1.27 27.94) (size 1 1) (drill 0.65) (layers "*.Cu" "*.Mask"))
  (pad "47" thru_hole oval (at 0 29.21) (size 1 1) (drill 0.65) (layers "*.Cu" "*.Mask"))
  (pad "48" thru_hole oval (at -1.27 29.21) (size 1 1) (drill 0.65) (layers "*.Cu" "*.Mask"))
  (pad "49" thru_hole oval (at 0 30.48) (size 1 1) (drill 0.65) (layers "*.Cu" "*.Mask"))
  (pad "50" thru_hole oval (at -1.27 30.48) (size 1 1) (drill 0.65) (layers "*.Cu" "*.Mask"))
  (pad "51" thru_hole oval (at 0 31.75) (size 1 1) (drill 0.65) (layers "*.Cu" "*.Mask"))
  (pad "52" thru_hole oval (at -1.27 31.75) (size 1 1) (drill 0.65) (layers "*.Cu" "*.Mask"))
  (pad "53" thru_hole oval (at 0 33.02) (size 1 1) (drill 0.65) (layers "*.Cu" "*.Mask"))
  (pad "54" thru_hole oval (at -1.27 33.02) (size 1 1) (drill 0.65) (layers "*.Cu" "*.Mask"))
  (pad "55" thru_hole oval (at 0 34.29) (size 1 1) (drill 0.65) (layers "*.Cu" "*.Mask"))
  (pad "56" thru_hole oval (at -1.27 34.29) (size 1 1) (drill 0.65) (layers "*.Cu" "*.Mask"))
  (pad "57" thru_hole oval (at 0 35.56) (size 1 1) (drill 0.65) (layers "*.Cu" "*.Mask"))
  (pad "58" thru_hole oval (at -1.27 35.56) (size 1 1) (drill 0.65) (layers "*.Cu" "*.Mask"))
  (pad "59" thru_hole oval (at 0 36.83) (size 1 1) (drill 0.65) (layers "*.Cu" "*.Mask"))
  (pad "60" thru_hole oval (at -1.27 36.83) (size 1 1) (drill 0.65) (layers "*.Cu" "*.Mask"))
  (pad "61" thru_hole oval (at 0 38.1) (size 1 1) (drill 0.65) (layers "*.Cu" "*.Mask"))
  (pad "62" thru_hole oval (at -1.27 38.1) (size 1 1) (drill 0.65) (layers "*.Cu" "*.Mask"))
  (pad "63" thru_hole oval (at 0 39.37) (size 1 1) (drill 0.65) (layers "*.Cu" "*.Mask"))
  (pad "64" thru_hole oval (at -1.27 39.37) (size 1 1) (drill 0.65) (layers "*.Cu" "*.Mask"))
  (pad "65" thru_hole oval (at 0 40.64) (size 1 1) (drill 0.65) (layers "*.Cu" "*.Mask"))
  (pad "66" thru_hole oval (at -1.27 40.64) (size 1 1) (drill 0.65) (layers "*.Cu" "*.Mask"))
  (pad "67" thru_hole oval (at 0 41.91) (size 1 1) (drill 0.65) (layers "*.Cu" "*.Mask"))
  (pad "68" thru_hole oval (at -1.27 41.91) (size 1 1) (drill 0.65) (layers "*.Cu" "*.Mask"))
  (pad "69" thru_hole oval (at 0 43.18) (size 1 1) (drill 0.65) (layers "*.Cu" "*.Mask"))
  (pad "70" thru_hole oval (at -1.27 43.18) (size 1 1) (drill 0.65) (layers "*.Cu" "*.Mask"))
  (pad "71" thru_hole oval (at 0 44.45) (size 1 1) (drill 0.65) (layers "*.Cu" "*.Mask"))
  (pad "72" thru_hole oval (at -1.27 44.45) (size 1 1) (drill 0.65) (layers "*.Cu" "*.Mask"))
  (pad "73" thru_hole oval (at 0 45.72) (size 1 1) (drill 0.65) (layers "*.Cu" "*.Mask"))
  (pad "74" thru_hole oval (at -1.27 45.72) (size 1 1) (drill 0.65) (layers "*.Cu" "*.Mask"))
  (pad "75" thru_hole oval (at 0 46.99) (size 1 1) (drill 0.65) (layers "*.Cu" "*.Mask"))
  (pad "76" thru_hole oval (at -1.27 46.99) (size 1 1) (drill 0.65) (layers "*.Cu" "*.Mask"))
  (pad "77" thru_hole oval (at 0 48.26) (size 1 1) (drill 0.65) (layers "*.Cu" "*.Mask"))
  (pad "78" thru_hole oval (at -1.27 48.26) (size 1 1) (drill 0.65) (layers "*.Cu" "*.Mask"))
  (pad "79" thru_hole oval (at 0 49.53) (size 1 1) (drill 0.65) (layers "*.Cu" "*.Mask"))
  (pad "80" thru_hole oval (at -1.27 49.53) (size 1 1) (drill 0.65) (layers "*.Cu" "*.Mask"))
  (pad "81" thru_hole oval (at 0 50.8) (size 1 1) (drill 0.65) (layers "*.Cu" "*.Mask"))
  (pad "82" thru_hole oval (at -1.27 50.8) (size 1 1) (drill 0.65) (layers "*.Cu" "*.Mask"))
  (pad "83" thru_hole oval (at 0 52.07) (size 1 1) (drill 0.65) (layers "*.Cu" "*.Mask"))
  (pad "84" thru_hole oval (at -1.27 52.07) (size 1 1) (drill 0.65) (layers "*.Cu" "*.Mask"))
  (pad "85" thru_hole oval (at 0 53.34) (size 1 1) (drill 0.65) (layers "*.Cu" "*.Mask"))
  (pad "86" thru_hole oval (at -1.27 53.34) (size 1 1) (drill 0.65) (layers "*.Cu" "*.Mask"))
  (pad "87" thru_hole oval (at 0 54.61) (size 1 1) (drill 0.65) (layers "*.Cu" "*.Mask"))
  (pad "88" thru_hole oval (at -1.27 54.61) (size 1 1) (drill 0.65) (layers "*.Cu" "*.Mask"))
  (pad "89" thru_hole oval (at 0 55.88) (size 1 1) (drill 0.65) (layers "*.Cu" "*.Mask"))
  (pad "90" thru_hole oval (at -1.27 55.88) (size 1 1) (drill 0.65) (layers "*.Cu" "*.Mask"))
  (pad "91" thru_hole oval (at 0 57.15) (size 1 1) (drill 0.65) (layers "*.Cu" "*.Mask"))
  (pad "92" thru_hole oval (at -1.27 57.15) (size 1 1) (drill 0.65) (layers "*.Cu" "*.Mask"))
  (pad "93" thru_hole oval (at 0 58.42) (size 1 1) (drill 0.65) (layers "*.Cu" "*.Mask"))
  (pad "94" thru_hole oval (at -1.27 58.42) (size 1 1) (drill 0.65) (layers "*.Cu" "*.Mask"))
  (pad "95" thru_hole oval (at 0 59.69) (size 1 1) (drill 0.65) (layers "*.Cu" "*.Mask"))
  (pad "96" thru_hole oval (at -1.27 59.69) (size 1 1) (drill 0.65) (layers "*.Cu" "*.Mask"))
  (pad "97" thru_hole oval (at 0 60.96) (size 1 1) (drill 0.65) (layers "*.Cu" "*.Mask"))
  (pad "98" thru_hole oval (at -1.27 60.96) (size 1 1) (drill 0.65) (layers "*.Cu" "*.Mask"))
  (pad "99" thru_hole oval (at 0 62.23) (size 1 1) (drill 0.65) (layers "*.Cu" "*.Mask"))
  (pad "100" thru_hole oval (at -1.27 62.23) (size 1 1) (drill 0.65) (layers "*.Cu" "*.Mask")))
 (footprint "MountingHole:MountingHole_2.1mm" (layer "F.Cu") (at 205.9 56.7)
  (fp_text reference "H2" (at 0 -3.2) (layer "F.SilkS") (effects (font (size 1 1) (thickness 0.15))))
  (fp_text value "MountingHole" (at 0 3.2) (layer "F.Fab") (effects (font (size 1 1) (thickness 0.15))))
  (pad "" np_thru_hole circle (at 0 0) (size 2.1 2.1) (drill 2.1) (layers "*.Cu" "*.Mask")))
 (gr_rect (start 91.9 51.3) (end 212 133.9) (stroke (width 0.1) (type default)) (fill none) (layer "Edge.Cuts"))
 (segment (start 145.22 106) (end 145.22 92.48) (width 0.25) (layer "F.Cu") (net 5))
 (segment (start 145.22 92.48) (end 145.9875 91.7125) (width 0.25) (layer "F.Cu") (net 5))
 (segment (start 154.228185 93.1) (end 153.190685 92.0625) (width 0.25) (layer "F.Cu") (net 2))
 (segment (start 148.659315 92.0625) (end 148.4 92.321815) (width 0.25) (layer "F.Cu") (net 2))
 (segment (start 148.4 92.321815) (end 148.4 93.125) (width 0.25) (layer "F.Cu") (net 2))
 (segment (start 157.225 90.103185) (end 154.228185 93.1) (width 0.25) (layer "F.Cu") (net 2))
 (segment (start 153.190685 92.0625) (end 148.659315 92.0625) (width 0.25) (layer "F.Cu") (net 2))
 (segment (start 157.225 66.1) (end 157.225 90.103185) (width 0.25) (layer "F.Cu") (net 2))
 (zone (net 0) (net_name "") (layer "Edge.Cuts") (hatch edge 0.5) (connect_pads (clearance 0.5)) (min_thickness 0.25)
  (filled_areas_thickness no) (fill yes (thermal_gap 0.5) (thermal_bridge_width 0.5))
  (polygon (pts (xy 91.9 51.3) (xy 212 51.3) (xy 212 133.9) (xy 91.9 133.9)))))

